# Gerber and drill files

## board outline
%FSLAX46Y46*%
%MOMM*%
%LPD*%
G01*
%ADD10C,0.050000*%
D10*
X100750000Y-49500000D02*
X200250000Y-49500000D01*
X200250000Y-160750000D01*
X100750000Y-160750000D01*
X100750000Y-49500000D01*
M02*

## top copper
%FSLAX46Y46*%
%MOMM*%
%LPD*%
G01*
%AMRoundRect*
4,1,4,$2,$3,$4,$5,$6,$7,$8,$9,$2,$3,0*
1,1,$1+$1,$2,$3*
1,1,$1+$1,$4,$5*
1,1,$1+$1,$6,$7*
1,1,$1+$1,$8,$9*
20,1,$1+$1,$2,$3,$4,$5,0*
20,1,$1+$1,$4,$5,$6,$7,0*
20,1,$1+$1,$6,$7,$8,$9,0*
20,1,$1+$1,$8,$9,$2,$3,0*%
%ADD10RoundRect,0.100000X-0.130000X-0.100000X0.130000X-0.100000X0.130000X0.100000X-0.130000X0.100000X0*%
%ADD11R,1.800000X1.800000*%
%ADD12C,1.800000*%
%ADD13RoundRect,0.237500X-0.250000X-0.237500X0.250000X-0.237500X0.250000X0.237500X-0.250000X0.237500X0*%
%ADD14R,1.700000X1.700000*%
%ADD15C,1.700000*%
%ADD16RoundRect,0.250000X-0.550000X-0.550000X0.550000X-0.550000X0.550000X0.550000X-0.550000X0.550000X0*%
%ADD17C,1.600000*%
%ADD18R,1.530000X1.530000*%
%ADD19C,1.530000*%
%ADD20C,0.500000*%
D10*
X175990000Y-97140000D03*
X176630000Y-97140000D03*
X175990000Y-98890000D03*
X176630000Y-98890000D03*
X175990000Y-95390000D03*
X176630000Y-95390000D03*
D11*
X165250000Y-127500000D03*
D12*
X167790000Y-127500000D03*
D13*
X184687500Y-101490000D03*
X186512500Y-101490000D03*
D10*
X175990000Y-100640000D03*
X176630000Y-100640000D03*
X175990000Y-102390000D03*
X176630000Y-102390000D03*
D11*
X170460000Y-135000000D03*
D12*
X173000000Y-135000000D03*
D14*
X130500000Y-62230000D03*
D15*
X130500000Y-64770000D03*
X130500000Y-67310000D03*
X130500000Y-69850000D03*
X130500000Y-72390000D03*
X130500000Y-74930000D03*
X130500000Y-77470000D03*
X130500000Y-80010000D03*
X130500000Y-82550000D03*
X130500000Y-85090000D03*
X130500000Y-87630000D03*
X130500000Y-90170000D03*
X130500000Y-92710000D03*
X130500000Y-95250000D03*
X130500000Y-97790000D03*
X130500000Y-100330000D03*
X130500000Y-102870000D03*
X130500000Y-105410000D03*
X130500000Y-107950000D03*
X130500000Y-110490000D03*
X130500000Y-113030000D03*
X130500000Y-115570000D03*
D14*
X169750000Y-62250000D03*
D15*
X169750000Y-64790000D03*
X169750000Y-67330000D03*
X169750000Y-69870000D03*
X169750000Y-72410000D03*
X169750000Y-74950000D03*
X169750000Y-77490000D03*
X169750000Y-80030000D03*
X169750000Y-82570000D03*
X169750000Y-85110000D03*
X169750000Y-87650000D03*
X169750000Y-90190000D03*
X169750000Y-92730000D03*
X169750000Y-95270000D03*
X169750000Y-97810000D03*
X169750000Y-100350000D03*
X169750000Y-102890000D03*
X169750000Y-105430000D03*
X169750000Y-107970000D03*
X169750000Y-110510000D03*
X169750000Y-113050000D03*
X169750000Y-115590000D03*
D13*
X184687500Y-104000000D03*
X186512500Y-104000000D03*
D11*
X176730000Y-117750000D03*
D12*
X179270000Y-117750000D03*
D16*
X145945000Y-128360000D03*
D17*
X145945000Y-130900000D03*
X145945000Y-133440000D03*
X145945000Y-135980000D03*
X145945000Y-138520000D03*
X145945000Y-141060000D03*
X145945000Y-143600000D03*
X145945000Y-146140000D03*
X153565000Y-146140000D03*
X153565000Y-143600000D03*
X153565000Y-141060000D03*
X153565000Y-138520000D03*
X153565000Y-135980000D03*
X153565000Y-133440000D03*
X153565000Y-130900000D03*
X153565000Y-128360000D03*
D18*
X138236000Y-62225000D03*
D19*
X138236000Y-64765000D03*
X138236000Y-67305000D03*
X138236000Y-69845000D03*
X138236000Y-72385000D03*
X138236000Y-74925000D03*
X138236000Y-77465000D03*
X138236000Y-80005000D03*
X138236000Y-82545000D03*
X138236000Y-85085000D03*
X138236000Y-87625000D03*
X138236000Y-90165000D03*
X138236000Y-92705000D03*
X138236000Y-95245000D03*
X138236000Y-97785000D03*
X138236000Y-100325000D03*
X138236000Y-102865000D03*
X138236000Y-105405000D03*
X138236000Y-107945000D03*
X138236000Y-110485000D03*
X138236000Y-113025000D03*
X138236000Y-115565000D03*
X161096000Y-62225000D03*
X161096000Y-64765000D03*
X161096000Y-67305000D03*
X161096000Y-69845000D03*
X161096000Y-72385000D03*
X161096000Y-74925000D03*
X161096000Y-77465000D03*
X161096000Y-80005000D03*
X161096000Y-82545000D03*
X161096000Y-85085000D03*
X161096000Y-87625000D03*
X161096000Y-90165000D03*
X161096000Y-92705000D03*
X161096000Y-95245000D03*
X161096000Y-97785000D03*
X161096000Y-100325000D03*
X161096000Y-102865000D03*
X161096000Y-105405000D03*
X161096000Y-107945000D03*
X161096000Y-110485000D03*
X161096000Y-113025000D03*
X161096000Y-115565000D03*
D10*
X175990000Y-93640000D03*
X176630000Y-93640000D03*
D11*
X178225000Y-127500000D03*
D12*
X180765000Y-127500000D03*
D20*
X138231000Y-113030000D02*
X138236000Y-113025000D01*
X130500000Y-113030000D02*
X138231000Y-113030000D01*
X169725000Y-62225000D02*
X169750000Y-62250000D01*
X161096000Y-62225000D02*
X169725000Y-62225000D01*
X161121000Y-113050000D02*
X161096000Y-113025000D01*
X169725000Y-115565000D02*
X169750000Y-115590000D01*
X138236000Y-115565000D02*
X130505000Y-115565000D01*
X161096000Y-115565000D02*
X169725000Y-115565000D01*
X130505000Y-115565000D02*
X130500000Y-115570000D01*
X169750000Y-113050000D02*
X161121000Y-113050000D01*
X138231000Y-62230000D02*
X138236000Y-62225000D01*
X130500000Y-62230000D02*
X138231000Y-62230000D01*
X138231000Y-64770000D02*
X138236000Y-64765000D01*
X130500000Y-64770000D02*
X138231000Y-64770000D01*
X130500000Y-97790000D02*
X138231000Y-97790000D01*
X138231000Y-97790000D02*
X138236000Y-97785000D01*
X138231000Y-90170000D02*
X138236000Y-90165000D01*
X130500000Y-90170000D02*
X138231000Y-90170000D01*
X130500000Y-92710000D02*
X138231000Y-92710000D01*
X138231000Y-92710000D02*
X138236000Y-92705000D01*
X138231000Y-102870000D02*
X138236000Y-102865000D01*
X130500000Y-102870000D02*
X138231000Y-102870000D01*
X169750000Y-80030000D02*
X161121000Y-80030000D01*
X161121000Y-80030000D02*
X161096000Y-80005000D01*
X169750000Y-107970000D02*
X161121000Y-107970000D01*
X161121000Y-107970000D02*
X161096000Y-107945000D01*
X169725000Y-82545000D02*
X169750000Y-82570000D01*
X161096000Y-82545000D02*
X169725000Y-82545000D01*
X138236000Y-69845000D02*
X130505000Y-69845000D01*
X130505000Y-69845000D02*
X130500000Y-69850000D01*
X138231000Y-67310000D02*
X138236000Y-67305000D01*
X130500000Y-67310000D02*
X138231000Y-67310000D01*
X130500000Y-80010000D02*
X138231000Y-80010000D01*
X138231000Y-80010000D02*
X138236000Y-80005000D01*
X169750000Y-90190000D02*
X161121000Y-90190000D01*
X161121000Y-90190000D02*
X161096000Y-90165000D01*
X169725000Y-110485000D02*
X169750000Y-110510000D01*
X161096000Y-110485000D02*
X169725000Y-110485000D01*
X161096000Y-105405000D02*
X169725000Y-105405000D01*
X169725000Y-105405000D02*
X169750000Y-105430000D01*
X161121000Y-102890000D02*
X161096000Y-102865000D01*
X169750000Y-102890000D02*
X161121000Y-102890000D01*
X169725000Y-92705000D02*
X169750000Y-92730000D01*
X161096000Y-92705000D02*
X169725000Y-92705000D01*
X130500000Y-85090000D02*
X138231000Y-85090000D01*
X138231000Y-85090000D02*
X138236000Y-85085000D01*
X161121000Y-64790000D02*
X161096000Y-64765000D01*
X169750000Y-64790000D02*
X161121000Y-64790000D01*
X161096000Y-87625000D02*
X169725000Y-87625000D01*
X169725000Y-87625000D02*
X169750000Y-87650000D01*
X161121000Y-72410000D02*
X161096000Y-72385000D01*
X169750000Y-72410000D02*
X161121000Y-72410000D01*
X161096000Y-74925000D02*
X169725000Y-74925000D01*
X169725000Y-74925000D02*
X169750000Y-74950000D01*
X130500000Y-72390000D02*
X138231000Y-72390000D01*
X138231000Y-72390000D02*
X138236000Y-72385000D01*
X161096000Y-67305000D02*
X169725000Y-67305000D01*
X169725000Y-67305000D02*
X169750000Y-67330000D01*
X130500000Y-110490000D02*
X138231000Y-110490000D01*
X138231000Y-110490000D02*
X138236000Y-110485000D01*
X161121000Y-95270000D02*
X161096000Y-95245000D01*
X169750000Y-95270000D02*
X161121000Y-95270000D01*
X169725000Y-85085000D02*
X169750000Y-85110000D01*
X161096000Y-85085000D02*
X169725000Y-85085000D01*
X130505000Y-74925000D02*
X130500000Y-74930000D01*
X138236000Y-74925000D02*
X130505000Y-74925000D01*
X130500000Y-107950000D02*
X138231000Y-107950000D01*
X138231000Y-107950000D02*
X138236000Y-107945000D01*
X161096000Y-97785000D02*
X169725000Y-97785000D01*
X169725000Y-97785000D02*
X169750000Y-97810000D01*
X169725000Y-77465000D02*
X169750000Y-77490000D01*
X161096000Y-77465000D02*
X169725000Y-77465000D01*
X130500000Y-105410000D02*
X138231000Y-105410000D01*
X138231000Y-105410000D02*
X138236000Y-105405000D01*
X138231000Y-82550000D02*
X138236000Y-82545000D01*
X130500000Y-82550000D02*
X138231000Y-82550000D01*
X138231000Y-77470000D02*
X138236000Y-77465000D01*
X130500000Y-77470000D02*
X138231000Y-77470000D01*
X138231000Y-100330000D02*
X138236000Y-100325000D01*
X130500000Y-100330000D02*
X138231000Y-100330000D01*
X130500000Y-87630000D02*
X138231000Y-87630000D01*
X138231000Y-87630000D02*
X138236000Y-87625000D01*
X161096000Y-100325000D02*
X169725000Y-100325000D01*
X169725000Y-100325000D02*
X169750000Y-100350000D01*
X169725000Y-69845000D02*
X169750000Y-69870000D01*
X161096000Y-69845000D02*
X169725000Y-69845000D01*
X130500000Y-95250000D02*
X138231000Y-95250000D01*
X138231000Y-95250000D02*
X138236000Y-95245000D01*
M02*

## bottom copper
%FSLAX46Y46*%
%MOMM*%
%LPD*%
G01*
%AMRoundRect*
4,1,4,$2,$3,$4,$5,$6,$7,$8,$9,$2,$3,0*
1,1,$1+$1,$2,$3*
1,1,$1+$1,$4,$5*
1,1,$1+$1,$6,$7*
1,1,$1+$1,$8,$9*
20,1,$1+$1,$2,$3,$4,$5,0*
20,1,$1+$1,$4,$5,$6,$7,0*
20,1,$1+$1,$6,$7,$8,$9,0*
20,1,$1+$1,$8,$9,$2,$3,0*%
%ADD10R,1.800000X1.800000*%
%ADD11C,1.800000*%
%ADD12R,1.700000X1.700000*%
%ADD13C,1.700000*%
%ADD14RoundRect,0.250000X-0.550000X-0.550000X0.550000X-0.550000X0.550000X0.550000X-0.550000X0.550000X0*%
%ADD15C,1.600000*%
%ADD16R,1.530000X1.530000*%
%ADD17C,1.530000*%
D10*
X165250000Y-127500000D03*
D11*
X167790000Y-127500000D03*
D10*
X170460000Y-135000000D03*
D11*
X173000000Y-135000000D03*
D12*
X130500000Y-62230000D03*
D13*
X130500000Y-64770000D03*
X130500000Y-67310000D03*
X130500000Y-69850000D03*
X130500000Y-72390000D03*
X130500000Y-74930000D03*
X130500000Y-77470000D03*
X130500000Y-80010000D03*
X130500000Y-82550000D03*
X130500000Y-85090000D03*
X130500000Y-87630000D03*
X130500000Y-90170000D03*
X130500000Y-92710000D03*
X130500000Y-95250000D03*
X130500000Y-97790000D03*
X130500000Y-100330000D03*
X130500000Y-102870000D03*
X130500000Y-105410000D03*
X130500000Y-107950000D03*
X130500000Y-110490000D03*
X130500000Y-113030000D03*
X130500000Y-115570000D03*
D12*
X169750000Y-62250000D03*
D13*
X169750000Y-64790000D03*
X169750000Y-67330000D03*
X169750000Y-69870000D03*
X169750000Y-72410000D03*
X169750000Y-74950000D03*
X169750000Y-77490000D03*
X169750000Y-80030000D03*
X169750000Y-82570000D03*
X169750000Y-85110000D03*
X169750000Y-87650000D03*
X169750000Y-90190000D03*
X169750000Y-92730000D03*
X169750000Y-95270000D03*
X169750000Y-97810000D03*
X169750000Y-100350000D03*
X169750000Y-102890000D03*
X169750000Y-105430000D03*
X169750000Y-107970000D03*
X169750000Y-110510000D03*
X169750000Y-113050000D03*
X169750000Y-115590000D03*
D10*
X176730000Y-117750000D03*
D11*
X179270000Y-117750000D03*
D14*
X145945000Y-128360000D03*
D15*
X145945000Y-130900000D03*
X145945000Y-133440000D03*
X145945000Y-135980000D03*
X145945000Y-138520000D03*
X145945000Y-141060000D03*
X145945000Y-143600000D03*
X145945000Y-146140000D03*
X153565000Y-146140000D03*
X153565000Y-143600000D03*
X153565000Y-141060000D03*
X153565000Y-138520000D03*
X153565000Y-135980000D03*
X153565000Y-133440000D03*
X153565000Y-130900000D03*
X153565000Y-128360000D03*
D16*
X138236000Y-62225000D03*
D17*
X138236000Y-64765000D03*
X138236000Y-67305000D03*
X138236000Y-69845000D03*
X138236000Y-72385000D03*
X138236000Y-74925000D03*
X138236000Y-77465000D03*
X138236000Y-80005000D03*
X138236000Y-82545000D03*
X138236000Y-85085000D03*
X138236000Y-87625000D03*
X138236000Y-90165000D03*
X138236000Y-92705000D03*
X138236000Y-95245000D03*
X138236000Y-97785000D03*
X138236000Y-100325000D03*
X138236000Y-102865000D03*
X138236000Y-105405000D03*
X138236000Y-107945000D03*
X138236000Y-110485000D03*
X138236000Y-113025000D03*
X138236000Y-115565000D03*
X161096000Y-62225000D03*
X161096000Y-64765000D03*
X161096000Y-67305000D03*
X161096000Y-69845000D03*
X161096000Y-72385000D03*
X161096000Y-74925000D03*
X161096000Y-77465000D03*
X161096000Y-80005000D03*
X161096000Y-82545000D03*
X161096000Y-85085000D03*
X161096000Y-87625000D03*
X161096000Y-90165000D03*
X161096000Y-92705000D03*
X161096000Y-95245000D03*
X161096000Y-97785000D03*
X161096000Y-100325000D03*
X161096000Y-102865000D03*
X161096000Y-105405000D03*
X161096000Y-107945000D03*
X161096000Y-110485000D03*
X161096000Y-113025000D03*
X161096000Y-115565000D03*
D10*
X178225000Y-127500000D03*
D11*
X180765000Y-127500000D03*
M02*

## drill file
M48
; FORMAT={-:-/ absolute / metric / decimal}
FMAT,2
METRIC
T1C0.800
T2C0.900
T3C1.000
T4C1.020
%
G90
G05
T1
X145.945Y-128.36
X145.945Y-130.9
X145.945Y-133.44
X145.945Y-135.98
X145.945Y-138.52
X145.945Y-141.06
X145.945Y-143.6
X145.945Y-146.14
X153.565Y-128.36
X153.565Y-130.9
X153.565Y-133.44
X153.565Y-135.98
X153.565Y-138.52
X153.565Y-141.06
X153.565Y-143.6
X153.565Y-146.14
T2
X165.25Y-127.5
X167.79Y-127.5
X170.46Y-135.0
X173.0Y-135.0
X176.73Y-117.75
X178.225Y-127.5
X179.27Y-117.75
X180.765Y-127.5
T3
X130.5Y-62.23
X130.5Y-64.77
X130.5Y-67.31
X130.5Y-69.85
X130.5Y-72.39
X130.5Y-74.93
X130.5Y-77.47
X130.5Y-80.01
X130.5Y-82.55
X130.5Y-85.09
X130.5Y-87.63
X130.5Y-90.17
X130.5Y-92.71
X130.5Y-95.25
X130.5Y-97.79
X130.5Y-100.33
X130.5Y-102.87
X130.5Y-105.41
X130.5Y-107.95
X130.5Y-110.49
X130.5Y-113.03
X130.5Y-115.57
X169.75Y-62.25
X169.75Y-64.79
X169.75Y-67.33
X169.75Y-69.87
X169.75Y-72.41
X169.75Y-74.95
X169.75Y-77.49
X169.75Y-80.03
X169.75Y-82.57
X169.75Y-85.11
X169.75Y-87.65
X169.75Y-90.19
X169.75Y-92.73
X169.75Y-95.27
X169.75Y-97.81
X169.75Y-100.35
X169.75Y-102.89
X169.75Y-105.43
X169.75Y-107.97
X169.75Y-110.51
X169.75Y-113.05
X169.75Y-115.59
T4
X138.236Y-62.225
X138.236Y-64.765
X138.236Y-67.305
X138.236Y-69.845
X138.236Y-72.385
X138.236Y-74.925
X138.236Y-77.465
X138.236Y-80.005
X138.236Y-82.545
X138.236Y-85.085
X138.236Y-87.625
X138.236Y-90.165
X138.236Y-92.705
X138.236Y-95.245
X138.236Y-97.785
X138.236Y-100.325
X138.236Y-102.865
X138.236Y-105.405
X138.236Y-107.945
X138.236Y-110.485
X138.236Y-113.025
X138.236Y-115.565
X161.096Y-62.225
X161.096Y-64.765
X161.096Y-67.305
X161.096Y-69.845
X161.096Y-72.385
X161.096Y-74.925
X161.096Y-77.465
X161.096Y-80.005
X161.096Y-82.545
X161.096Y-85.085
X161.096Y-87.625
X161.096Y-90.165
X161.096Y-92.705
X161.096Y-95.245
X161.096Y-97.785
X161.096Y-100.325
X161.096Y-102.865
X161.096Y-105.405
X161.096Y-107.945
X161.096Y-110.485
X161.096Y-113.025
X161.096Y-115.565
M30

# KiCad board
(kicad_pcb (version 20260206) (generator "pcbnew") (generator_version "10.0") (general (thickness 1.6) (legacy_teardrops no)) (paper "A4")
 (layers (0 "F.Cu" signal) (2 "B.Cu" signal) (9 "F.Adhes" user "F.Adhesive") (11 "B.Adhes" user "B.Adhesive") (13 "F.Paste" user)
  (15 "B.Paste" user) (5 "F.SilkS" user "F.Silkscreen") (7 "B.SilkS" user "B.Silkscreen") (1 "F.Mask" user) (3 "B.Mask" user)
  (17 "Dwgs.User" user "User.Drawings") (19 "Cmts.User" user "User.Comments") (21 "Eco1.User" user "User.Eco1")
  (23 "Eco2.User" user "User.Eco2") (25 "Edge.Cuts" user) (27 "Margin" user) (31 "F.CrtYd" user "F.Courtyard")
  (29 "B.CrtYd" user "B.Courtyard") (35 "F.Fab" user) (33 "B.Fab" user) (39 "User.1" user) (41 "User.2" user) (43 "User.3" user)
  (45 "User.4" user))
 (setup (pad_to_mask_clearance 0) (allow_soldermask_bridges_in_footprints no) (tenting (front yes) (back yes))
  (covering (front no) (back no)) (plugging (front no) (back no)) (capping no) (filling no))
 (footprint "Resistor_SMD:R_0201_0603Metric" (layer "F.Cu") (at 176.31 97.14)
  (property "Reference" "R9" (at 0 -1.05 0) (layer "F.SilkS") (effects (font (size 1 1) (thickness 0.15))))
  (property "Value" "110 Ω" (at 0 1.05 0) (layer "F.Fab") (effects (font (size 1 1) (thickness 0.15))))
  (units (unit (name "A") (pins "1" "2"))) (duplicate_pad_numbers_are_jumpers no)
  (pad "" smd roundrect (at -0.345 0) (size 0.318 0.36) (layers "F.Paste") (roundrect_rratio 0.25))
  (pad "" smd roundrect (at 0.345 0) (size 0.318 0.36) (layers "F.Paste") (roundrect_rratio 0.25))
  (pad "1" smd roundrect (at -0.32 0) (size 0.46 0.4) (layers "F.Cu" "F.Mask") (roundrect_rratio 0.25) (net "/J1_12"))
  (pad "2" smd roundrect (at 0.32 0) (size 0.46 0.4) (layers "F.Cu" "F.Mask") (roundrect_rratio 0.25) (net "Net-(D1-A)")))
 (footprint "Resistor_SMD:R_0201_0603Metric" (layer "F.Cu") (at 176.31 98.89)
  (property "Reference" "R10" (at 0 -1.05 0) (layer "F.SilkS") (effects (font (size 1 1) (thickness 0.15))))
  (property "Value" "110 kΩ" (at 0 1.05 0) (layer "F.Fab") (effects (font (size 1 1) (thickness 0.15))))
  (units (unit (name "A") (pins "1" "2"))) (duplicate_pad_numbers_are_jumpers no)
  (pad "" smd roundrect (at -0.345 0) (size 0.318 0.36) (layers "F.Paste") (roundrect_rratio 0.25))
  (pad "" smd roundrect (at 0.345 0) (size 0.318 0.36) (layers "F.Paste") (roundrect_rratio 0.25))
  (pad "1" smd roundrect (at -0.32 0) (size 0.46 0.4) (layers "F.Cu" "F.Mask") (roundrect_rratio 0.25) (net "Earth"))
  (pad "2" smd roundrect (at 0.32 0) (size 0.46 0.4) (layers "F.Cu" "F.Mask") (roundrect_rratio 0.25) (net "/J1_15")))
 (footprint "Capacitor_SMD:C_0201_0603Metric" (layer "F.Cu") (at 176.31 95.39)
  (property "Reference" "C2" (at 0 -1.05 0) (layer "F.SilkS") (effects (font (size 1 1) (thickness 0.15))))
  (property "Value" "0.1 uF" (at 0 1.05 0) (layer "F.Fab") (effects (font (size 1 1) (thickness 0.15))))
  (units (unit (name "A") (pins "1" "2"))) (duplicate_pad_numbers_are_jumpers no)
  (pad "" smd roundrect (at -0.345 0) (size 0.318 0.36) (layers "F.Paste") (roundrect_rratio 0.25))
  (pad "" smd roundrect (at 0.345 0) (size 0.318 0.36) (layers "F.Paste") (roundrect_rratio 0.25))
  (pad "1" smd roundrect (at -0.32 0) (size 0.46 0.4) (layers "F.Cu" "F.Mask") (roundrect_rratio 0.25) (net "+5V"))
  (pad "2" smd roundrect (at 0.32 0) (size 0.46 0.4) (layers "F.Cu" "F.Mask") (roundrect_rratio 0.25) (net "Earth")))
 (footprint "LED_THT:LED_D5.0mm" (layer "F.Cu") (at 165.25 127.5)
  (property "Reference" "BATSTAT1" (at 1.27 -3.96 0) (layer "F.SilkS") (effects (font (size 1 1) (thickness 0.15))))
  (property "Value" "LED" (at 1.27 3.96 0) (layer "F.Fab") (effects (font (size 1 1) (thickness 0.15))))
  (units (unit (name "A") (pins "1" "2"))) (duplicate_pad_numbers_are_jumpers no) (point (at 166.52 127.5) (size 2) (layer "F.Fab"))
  (pad "1" thru_hole rect (at 0 0) (size 1.8 1.8) (drill 0.9) (layers "*.Cu" "*.Mask") (remove_unused_layers no) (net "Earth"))
  (pad "2" thru_hole circle (at 2.54 0) (size 1.8 1.8) (drill 0.9) (layers "*.Cu" "*.Mask") (remove_unused_layers no)
   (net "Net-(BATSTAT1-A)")))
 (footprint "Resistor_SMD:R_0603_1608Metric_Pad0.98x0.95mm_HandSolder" (layer "F.Cu") (at 185.6 101.49)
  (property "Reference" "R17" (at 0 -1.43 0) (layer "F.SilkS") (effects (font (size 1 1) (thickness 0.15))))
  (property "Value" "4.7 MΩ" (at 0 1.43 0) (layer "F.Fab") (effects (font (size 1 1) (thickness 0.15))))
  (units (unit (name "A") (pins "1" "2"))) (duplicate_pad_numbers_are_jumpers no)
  (pad "1" smd roundrect (at -0.9125 0) (size 0.975 0.95) (layers "F.Cu" "F.Mask" "F.Paste") (roundrect_rratio 0.25) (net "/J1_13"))
  (pad "2" smd roundrect (at 0.9125 0) (size 0.975 0.95) (layers "F.Cu" "F.Mask" "F.Paste") (roundrect_rratio 0.25) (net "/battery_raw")))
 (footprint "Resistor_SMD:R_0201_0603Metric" (layer "F.Cu") (at 176.31 100.64)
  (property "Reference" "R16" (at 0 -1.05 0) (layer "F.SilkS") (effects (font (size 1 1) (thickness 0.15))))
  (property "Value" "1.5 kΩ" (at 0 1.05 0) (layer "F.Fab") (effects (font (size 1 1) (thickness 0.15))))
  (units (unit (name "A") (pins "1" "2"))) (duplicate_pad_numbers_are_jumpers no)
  (pad "" smd roundrect (at -0.345 0) (size 0.318 0.36) (layers "F.Paste") (roundrect_rratio 0.25))
  (pad "" smd roundrect (at 0.345 0) (size 0.318 0.36) (layers "F.Paste") (roundrect_rratio 0.25))
  (pad "1" smd roundrect (at -0.32 0) (size 0.46 0.4) (layers "F.Cu" "F.Mask") (roundrect_rratio 0.25) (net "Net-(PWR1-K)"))
  (pad "2" smd roundrect (at 0.32 0) (size 0.46 0.4) (layers "F.Cu" "F.Mask") (roundrect_rratio 0.25) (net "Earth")))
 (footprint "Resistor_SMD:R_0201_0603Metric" (layer "F.Cu") (at 176.31 102.39)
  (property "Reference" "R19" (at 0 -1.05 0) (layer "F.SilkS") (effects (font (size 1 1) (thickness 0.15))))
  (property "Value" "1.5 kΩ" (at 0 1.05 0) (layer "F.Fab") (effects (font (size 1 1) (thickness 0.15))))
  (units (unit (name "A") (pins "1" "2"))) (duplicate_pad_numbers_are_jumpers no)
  (pad "" smd roundrect (at -0.345 0) (size 0.318 0.36) (layers "F.Paste") (roundrect_rratio 0.25))
  (pad "" smd roundrect (at 0.345 0) (size 0.318 0.36) (layers "F.Paste") (roundrect_rratio 0.25))
  (pad "1" smd roundrect (at -0.32 0) (size 0.46 0.4) (layers "F.Cu" "F.Mask") (roundrect_rratio 0.25) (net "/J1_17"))
  (pad "2" smd roundrect (at 0.32 0) (size 0.46 0.4) (layers "F.Cu" "F.Mask") (roundrect_rratio 0.25) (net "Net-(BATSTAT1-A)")))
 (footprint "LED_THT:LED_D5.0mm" (layer "F.Cu") (at 170.46 135)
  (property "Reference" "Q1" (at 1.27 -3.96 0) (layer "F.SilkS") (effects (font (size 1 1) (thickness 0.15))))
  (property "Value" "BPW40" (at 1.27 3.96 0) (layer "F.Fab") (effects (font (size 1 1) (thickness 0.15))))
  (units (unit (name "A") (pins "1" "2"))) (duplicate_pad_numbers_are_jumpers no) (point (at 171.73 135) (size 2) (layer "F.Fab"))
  (pad "1" thru_hole rect (at 0 0) (size 1.8 1.8) (drill 0.9) (layers "*.Cu" "*.Mask") (remove_unused_layers no) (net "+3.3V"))
  (pad "2" thru_hole circle (at 2.54 0) (size 1.8 1.8) (drill 0.9) (layers "*.Cu" "*.Mask") (remove_unused_layers no) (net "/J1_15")))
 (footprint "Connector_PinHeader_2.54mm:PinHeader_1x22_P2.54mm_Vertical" (layer "F.Cu") (at 130.5 62.23)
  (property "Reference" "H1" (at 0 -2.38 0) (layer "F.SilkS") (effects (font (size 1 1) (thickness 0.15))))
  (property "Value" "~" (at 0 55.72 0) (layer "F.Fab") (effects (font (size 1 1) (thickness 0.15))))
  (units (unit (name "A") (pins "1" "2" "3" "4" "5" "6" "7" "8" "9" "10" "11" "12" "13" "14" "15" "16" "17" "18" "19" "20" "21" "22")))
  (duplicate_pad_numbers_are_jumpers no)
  (pad "1" thru_hole rect (at 0 0) (size 1.7 1.7) (drill 1) (layers "*.Cu" "*.Mask") (remove_unused_layers no) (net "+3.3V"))
  (pad "2" thru_hole circle (at 0 2.54) (size 1.7 1.7) (drill 1) (layers "*.Cu" "*.Mask") (remove_unused_layers no) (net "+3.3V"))
  (pad "3" thru_hole circle (at 0 5.08) (size 1.7 1.7) (drill 1) (layers "*.Cu" "*.Mask") (remove_unused_layers no) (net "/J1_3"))
  (pad "4" thru_hole circle (at 0 7.62) (size 1.7 1.7) (drill 1) (layers "*.Cu" "*.Mask") (remove_unused_layers no) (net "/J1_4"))
  (pad "5" thru_hole circle (at 0 10.16) (size 1.7 1.7) (drill 1) (layers "*.Cu" "*.Mask") (remove_unused_layers no) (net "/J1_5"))
  (pad "6" thru_hole circle (at 0 12.7) (size 1.7 1.7) (drill 1) (layers "*.Cu" "*.Mask") (remove_unused_layers no) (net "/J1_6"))
  (pad "7" thru_hole circle (at 0 15.24) (size 1.7 1.7) (drill 1) (layers "*.Cu" "*.Mask") (remove_unused_layers no) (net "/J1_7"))
  (pad "8" thru_hole circle (at 0 17.78) (size 1.7 1.7) (drill 1) (layers "*.Cu" "*.Mask") (remove_unused_layers no) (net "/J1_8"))
  (pad "9" thru_hole circle (at 0 20.32) (size 1.7 1.7) (drill 1) (layers "*.Cu" "*.Mask") (remove_unused_layers no) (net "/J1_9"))
  (pad "10" thru_hole circle (at 0 22.86) (size 1.7 1.7) (drill 1) (layers "*.Cu" "*.Mask") (remove_unused_layers no) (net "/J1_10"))
  (pad "11" thru_hole circle (at 0 25.4) (size 1.7 1.7) (drill 1) (layers "*.Cu" "*.Mask") (remove_unused_layers no) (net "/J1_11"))
  (pad "12" thru_hole circle (at 0 27.94) (size 1.7 1.7) (drill 1) (layers "*.Cu" "*.Mask") (remove_unused_layers no) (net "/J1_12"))
  (pad "13" thru_hole circle (at 0 30.48) (size 1.7 1.7) (drill 1) (layers "*.Cu" "*.Mask") (remove_unused_layers no) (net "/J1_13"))
  (pad "14" thru_hole circle (at 0 33.02) (size 1.7 1.7) (drill 1) (layers "*.Cu" "*.Mask") (remove_unused_layers no) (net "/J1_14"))
  (pad "15" thru_hole circle (at 0 35.56) (size 1.7 1.7) (drill 1) (layers "*.Cu" "*.Mask") (remove_unused_layers no) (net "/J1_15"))
  (pad "16" thru_hole circle (at 0 38.1) (size 1.7 1.7) (drill 1) (layers "*.Cu" "*.Mask") (remove_unused_layers no) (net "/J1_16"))
  (pad "17" thru_hole circle (at 0 40.64) (size 1.7 1.7) (drill 1) (layers "*.Cu" "*.Mask") (remove_unused_layers no) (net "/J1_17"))
  (pad "18" thru_hole circle (at 0 43.18) (size 1.7 1.7) (drill 1) (layers "*.Cu" "*.Mask") (remove_unused_layers no) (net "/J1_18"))
  (pad "19" thru_hole circle (at 0 45.72) (size 1.7 1.7) (drill 1) (layers "*.Cu" "*.Mask") (remove_unused_layers no) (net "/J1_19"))
  (pad "20" thru_hole circle (at 0 48.26) (size 1.7 1.7) (drill 1) (layers "*.Cu" "*.Mask") (remove_unused_layers no) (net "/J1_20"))
  (pad "21" thru_hole circle (at 0 50.8) (size 1.7 1.7) (drill 1) (layers "*.Cu" "*.Mask") (remove_unused_layers no) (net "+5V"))
  (pad "22" thru_hole circle (at 0 53.34) (size 1.7 1.7) (drill 1) (layers "*.Cu" "*.Mask") (remove_unused_layers no) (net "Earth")))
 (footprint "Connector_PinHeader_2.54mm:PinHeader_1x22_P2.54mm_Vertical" (layer "F.Cu") (at 169.75 62.25)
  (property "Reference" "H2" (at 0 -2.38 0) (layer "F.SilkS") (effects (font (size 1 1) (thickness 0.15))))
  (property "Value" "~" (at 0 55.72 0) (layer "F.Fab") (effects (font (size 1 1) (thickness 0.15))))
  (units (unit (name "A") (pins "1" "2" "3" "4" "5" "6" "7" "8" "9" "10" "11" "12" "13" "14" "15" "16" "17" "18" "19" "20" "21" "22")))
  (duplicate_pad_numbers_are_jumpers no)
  (pad "1" thru_hole rect (at 0 0) (size 1.7 1.7) (drill 1) (layers "*.Cu" "*.Mask") (remove_unused_layers no) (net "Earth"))
  (pad "2" thru_hole circle (at 0 2.54) (size 1.7 1.7) (drill 1) (layers "*.Cu" "*.Mask") (remove_unused_layers no) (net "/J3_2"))
  (pad "3" thru_hole circle (at 0 5.08) (size 1.7 1.7) (drill 1) (layers "*.Cu" "*.Mask") (remove_unused_layers no) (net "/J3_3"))
  (pad "4" thru_hole circle (at 0 7.62) (size 1.7 1.7) (drill 1) (layers "*.Cu" "*.Mask") (remove_unused_layers no) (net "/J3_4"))
  (pad "5" thru_hole circle (at 0 10.16) (size 1.7 1.7) (drill 1) (layers "*.Cu" "*.Mask") (remove_unused_layers no) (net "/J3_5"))
  (pad "6" thru_hole circle (at 0 12.7) (size 1.7 1.7) (drill 1) (layers "*.Cu" "*.Mask") (remove_unused_layers no) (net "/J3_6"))
  (pad "7" thru_hole circle (at 0 15.24) (size 1.7 1.7) (drill 1) (layers "*.Cu" "*.Mask") (remove_unused_layers no) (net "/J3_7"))
  (pad "8" thru_hole circle (at 0 17.78) (size 1.7 1.7) (drill 1) (layers "*.Cu" "*.Mask") (remove_unused_layers no) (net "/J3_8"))
  (pad "9" thru_hole circle (at 0 20.32) (size 1.7 1.7) (drill 1) (layers "*.Cu" "*.Mask") (remove_unused_layers no) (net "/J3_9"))
  (pad "10" thru_hole circle (at 0 22.86) (size 1.7 1.7) (drill 1) (layers "*.Cu" "*.Mask") (remove_unused_layers no) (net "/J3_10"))
  (pad "11" thru_hole circle (at 0 25.4) (size 1.7 1.7) (drill 1) (layers "*.Cu" "*.Mask") (remove_unused_layers no) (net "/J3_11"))
  (pad "12" thru_hole circle (at 0 27.94) (size 1.7 1.7) (drill 1) (layers "*.Cu" "*.Mask") (remove_unused_layers no) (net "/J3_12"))
  (pad "13" thru_hole circle (at 0 30.48) (size 1.7 1.7) (drill 1) (layers "*.Cu" "*.Mask") (remove_unused_layers no) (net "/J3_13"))
  (pad "14" thru_hole circle (at 0 33.02) (size 1.7 1.7) (drill 1) (layers "*.Cu" "*.Mask") (remove_unused_layers no) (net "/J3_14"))
  (pad "15" thru_hole circle (at 0 35.56) (size 1.7 1.7) (drill 1) (layers "*.Cu" "*.Mask") (remove_unused_layers no) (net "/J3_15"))
  (pad "16" thru_hole circle (at 0 38.1) (size 1.7 1.7) (drill 1) (layers "*.Cu" "*.Mask") (remove_unused_layers no) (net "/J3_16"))
  (pad "17" thru_hole circle (at 0 40.64) (size 1.7 1.7) (drill 1) (layers "*.Cu" "*.Mask") (remove_unused_layers no) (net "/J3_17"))
  (pad "18" thru_hole circle (at 0 43.18) (size 1.7 1.7) (drill 1) (layers "*.Cu" "*.Mask") (remove_unused_layers no) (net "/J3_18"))
  (pad "19" thru_hole circle (at 0 45.72) (size 1.7 1.7) (drill 1) (layers "*.Cu" "*.Mask") (remove_unused_layers no) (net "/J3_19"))
  (pad "20" thru_hole circle (at 0 48.26) (size 1.7 1.7) (drill 1) (layers "*.Cu" "*.Mask") (remove_unused_layers no) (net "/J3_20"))
  (pad "21" thru_hole circle (at 0 50.8) (size 1.7 1.7) (drill 1) (layers "*.Cu" "*.Mask") (remove_unused_layers no) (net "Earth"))
  (pad "22" thru_hole circle (at 0 53.34) (size 1.7 1.7) (drill 1) (layers "*.Cu" "*.Mask") (remove_unused_layers no) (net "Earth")))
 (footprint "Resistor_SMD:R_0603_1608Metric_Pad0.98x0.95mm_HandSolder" (layer "F.Cu") (at 185.6 104)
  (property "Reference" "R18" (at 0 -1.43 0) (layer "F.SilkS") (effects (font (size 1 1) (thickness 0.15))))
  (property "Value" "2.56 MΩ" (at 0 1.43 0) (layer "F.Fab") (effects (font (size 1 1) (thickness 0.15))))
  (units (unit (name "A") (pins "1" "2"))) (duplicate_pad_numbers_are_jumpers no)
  (pad "1" smd roundrect (at -0.9125 0) (size 0.975 0.95) (layers "F.Cu" "F.Mask" "F.Paste") (roundrect_rratio 0.25) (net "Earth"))
  (pad "2" smd roundrect (at 0.9125 0) (size 0.975 0.95) (layers "F.Cu" "F.Mask" "F.Paste") (roundrect_rratio 0.25) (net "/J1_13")))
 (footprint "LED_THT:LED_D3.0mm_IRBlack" (layer "F.Cu") (at 176.73 117.75)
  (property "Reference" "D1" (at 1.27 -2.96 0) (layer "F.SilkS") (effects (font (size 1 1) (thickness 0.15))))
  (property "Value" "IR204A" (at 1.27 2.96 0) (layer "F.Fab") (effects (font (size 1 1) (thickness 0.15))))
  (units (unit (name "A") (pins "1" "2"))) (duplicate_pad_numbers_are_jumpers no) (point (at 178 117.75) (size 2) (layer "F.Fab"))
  (pad "1" thru_hole rect (at 0 0) (size 1.8 1.8) (drill 0.9) (layers "*.Cu" "*.Mask") (remove_unused_layers no) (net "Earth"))
  (pad "2" thru_hole circle (at 2.54 0) (size 1.8 1.8) (drill 0.9) (layers "*.Cu" "*.Mask") (remove_unused_layers no) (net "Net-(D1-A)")))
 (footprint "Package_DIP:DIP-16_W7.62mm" (layer "F.Cu") (at 145.945 128.36)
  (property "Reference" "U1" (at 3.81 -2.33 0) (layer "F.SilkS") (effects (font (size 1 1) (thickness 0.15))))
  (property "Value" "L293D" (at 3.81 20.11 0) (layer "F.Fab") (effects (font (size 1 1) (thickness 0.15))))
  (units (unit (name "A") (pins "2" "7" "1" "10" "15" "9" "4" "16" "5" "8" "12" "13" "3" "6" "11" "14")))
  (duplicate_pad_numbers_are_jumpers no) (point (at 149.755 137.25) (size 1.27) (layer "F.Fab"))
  (pad "1" thru_hole roundrect (at 0 0) (size 1.6 1.6) (drill 0.8) (layers "*.Cu" "*.Mask") (remove_unused_layers no)
   (roundrect_rratio 0.15625) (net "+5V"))
  (pad "2" thru_hole circle (at 0 2.54) (size 1.6 1.6) (drill 0.8) (layers "*.Cu" "*.Mask") (remove_unused_layers no) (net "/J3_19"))
  (pad "3" thru_hole circle (at 0 5.08) (size 1.6 1.6) (drill 0.8) (layers "*.Cu" "*.Mask") (remove_unused_layers no)
   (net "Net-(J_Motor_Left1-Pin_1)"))
  (pad "4" thru_hole circle (at 0 7.62) (size 1.6 1.6) (drill 0.8) (layers "*.Cu" "*.Mask") (remove_unused_layers no) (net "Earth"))
  (pad "5" thru_hole circle (at 0 10.16) (size 1.6 1.6) (drill 0.8) (layers "*.Cu" "*.Mask") (remove_unused_layers no) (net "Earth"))
  (pad "6" thru_hole circle (at 0 12.7) (size 1.6 1.6) (drill 0.8) (layers "*.Cu" "*.Mask") (remove_unused_layers no)
   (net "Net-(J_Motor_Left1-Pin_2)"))
  (pad "7" thru_hole circle (at 0 15.24) (size 1.6 1.6) (drill 0.8) (layers "*.Cu" "*.Mask") (remove_unused_layers no) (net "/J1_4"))
  (pad "8" thru_hole circle (at 0 17.78) (size 1.6 1.6) (drill 0.8) (layers "*.Cu" "*.Mask") (remove_unused_layers no) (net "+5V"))
  (pad "9" thru_hole circle (at 7.62 17.78) (size 1.6 1.6) (drill 0.8) (layers "*.Cu" "*.Mask") (remove_unused_layers no) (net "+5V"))
  (pad "10" thru_hole circle (at 7.62 15.24) (size 1.6 1.6) (drill 0.8) (layers "*.Cu" "*.Mask") (remove_unused_layers no) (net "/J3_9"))
  (pad "11" thru_hole circle (at 7.62 12.7) (size 1.6 1.6) (drill 0.8) (layers "*.Cu" "*.Mask") (remove_unused_layers no)
   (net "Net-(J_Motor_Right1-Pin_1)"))
  (pad "12" thru_hole circle (at 7.62 10.16) (size 1.6 1.6) (drill 0.8) (layers "*.Cu" "*.Mask") (remove_unused_layers no) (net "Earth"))
  (pad "13" thru_hole circle (at 7.62 7.62) (size 1.6 1.6) (drill 0.8) (layers "*.Cu" "*.Mask") (remove_unused_layers no) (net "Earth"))
  (pad "14" thru_hole circle (at 7.62 5.08) (size 1.6 1.6) (drill 0.8) (layers "*.Cu" "*.Mask") (remove_unused_layers no)
   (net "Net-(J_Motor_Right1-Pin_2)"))
  (pad "15" thru_hole circle (at 7.62 2.54) (size 1.6 1.6) (drill 0.8) (layers "*.Cu" "*.Mask") (remove_unused_layers no) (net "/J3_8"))
  (pad "16" thru_hole circle (at 7.62 0) (size 1.6 1.6) (drill 0.8) (layers "*.Cu" "*.Mask") (remove_unused_layers no) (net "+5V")))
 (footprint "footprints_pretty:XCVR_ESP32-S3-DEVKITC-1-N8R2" (layer "F.Cu") (at 149.666 92.195)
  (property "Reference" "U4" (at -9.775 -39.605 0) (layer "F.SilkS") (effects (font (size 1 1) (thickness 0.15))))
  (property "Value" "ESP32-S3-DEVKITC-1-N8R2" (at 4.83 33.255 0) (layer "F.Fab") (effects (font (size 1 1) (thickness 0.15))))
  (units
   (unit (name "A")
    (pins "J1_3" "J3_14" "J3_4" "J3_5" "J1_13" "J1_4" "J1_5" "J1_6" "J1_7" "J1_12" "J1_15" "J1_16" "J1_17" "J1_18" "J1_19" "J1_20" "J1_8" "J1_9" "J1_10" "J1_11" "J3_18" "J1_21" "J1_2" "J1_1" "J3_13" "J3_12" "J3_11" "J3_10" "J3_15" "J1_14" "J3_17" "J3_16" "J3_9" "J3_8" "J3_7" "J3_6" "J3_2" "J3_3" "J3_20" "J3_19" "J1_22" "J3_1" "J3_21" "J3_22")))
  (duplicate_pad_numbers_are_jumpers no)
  (pad "J1_1" thru_hole rect (at -11.43 -29.97) (size 1.53 1.53) (drill 1.02) (layers "*.Cu" "*.Mask") (remove_unused_layers no)
   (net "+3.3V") (solder_mask_margin 0.102))
  (pad "J1_2" thru_hole circle (at -11.43 -27.43) (size 1.53 1.53) (drill 1.02) (layers "*.Cu" "*.Mask") (remove_unused_layers no)
   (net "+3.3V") (solder_mask_margin 0.102))
  (pad "J1_3" thru_hole circle (at -11.43 -24.89) (size 1.53 1.53) (drill 1.02) (layers "*.Cu" "*.Mask") (remove_unused_layers no)
   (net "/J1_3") (solder_mask_margin 0.102))
  (pad "J1_4" thru_hole circle (at -11.43 -22.35) (size 1.53 1.53) (drill 1.02) (layers "*.Cu" "*.Mask") (remove_unused_layers no)
   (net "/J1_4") (solder_mask_margin 0.102))
  (pad "J1_5" thru_hole circle (at -11.43 -19.81) (size 1.53 1.53) (drill 1.02) (layers "*.Cu" "*.Mask") (remove_unused_layers no)
   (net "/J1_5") (solder_mask_margin 0.102))
  (pad "J1_6" thru_hole circle (at -11.43 -17.27) (size 1.53 1.53) (drill 1.02) (layers "*.Cu" "*.Mask") (remove_unused_layers no)
   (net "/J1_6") (solder_mask_margin 0.102))
  (pad "J1_7" thru_hole circle (at -11.43 -14.73) (size 1.53 1.53) (drill 1.02) (layers "*.Cu" "*.Mask") (remove_unused_layers no)
   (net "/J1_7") (solder_mask_margin 0.102))
  (pad "J1_8" thru_hole circle (at -11.43 -12.19) (size 1.53 1.53) (drill 1.02) (layers "*.Cu" "*.Mask") (remove_unused_layers no)
   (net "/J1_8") (solder_mask_margin 0.102))
  (pad "J1_9" thru_hole circle (at -11.43 -9.65) (size 1.53 1.53) (drill 1.02) (layers "*.Cu" "*.Mask") (remove_unused_layers no)
   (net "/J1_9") (solder_mask_margin 0.102))
  (pad "J1_10" thru_hole circle (at -11.43 -7.11) (size 1.53 1.53) (drill 1.02) (layers "*.Cu" "*.Mask") (remove_unused_layers no)
   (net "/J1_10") (solder_mask_margin 0.102))
  (pad "J1_11" thru_hole circle (at -11.43 -4.57) (size 1.53 1.53) (drill 1.02) (layers "*.Cu" "*.Mask") (remove_unused_layers no)
   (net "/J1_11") (solder_mask_margin 0.102))
  (pad "J1_12" thru_hole circle (at -11.43 -2.03) (size 1.53 1.53) (drill 1.02) (layers "*.Cu" "*.Mask") (remove_unused_layers no)
   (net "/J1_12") (solder_mask_margin 0.102))
  (pad "J1_13" thru_hole circle (at -11.43 0.51) (size 1.53 1.53) (drill 1.02) (layers "*.Cu" "*.Mask") (remove_unused_layers no)
   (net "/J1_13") (solder_mask_margin 0.102))
  (pad "J1_14" thru_hole circle (at -11.43 3.05) (size 1.53 1.53) (drill 1.02) (layers "*.Cu" "*.Mask") (remove_unused_layers no)
   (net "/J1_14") (solder_mask_margin 0.102))
  (pad "J1_15" thru_hole circle (at -11.43 5.59) (size 1.53 1.53) (drill 1.02) (layers "*.Cu" "*.Mask") (remove_unused_layers no)
   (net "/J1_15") (solder_mask_margin 0.102))
  (pad "J1_16" thru_hole circle (at -11.43 8.13) (size 1.53 1.53) (drill 1.02) (layers "*.Cu" "*.Mask") (remove_unused_layers no)
   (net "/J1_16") (solder_mask_margin 0.102))
  (pad "J1_17" thru_hole circle (at -11.43 10.67) (size 1.53 1.53) (drill 1.02) (layers "*.Cu" "*.Mask") (remove_unused_layers no)
   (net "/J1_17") (solder_mask_margin 0.102))
  (pad "J1_18" thru_hole circle (at -11.43 13.21) (size 1.53 1.53) (drill 1.02) (layers "*.Cu" "*.Mask") (remove_unused_layers no)
   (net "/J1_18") (solder_mask_margin 0.102))
  (pad "J1_19" thru_hole circle (at -11.43 15.75) (size 1.53 1.53) (drill 1.02) (layers "*.Cu" "*.Mask") (remove_unused_layers no)
   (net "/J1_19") (solder_mask_margin 0.102))
  (pad "J1_20" thru_hole circle (at -11.43 18.29) (size 1.53 1.53) (drill 1.02) (layers "*.Cu" "*.Mask") (remove_unused_layers no)
   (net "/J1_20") (solder_mask_margin 0.102))
  (pad "J1_21" thru_hole circle (at -11.43 20.83) (size 1.53 1.53) (drill 1.02) (layers "*.Cu" "*.Mask") (remove_unused_layers no)
   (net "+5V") (solder_mask_margin 0.102))
  (pad "J1_22" thru_hole circle (at -11.43 23.37) (size 1.53 1.53) (drill 1.02) (layers "*.Cu" "*.Mask") (remove_unused_layers no)
   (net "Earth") (solder_mask_margin 0.102))
  (pad "J3_1" thru_hole circle (at 11.43 -29.97) (size 1.53 1.53) (drill 1.02) (layers "*.Cu" "*.Mask") (remove_unused_layers no)
   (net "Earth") (solder_mask_margin 0.102))
  (pad "J3_2" thru_hole circle (at 11.43 -27.43) (size 1.53 1.53) (drill 1.02) (layers "*.Cu" "*.Mask") (remove_unused_layers no)
   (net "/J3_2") (solder_mask_margin 0.102))
  (pad "J3_3" thru_hole circle (at 11.43 -24.89) (size 1.53 1.53) (drill 1.02) (layers "*.Cu" "*.Mask") (remove_unused_layers no)
   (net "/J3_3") (solder_mask_margin 0.102))
  (pad "J3_4" thru_hole circle (at 11.43 -22.35) (size 1.53 1.53) (drill 1.02) (layers "*.Cu" "*.Mask") (remove_unused_layers no)
   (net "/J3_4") (solder_mask_margin 0.102))
  (pad "J3_5" thru_hole circle (at 11.43 -19.81) (size 1.53 1.53) (drill 1.02) (layers "*.Cu" "*.Mask") (remove_unused_layers no)
   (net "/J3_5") (solder_mask_margin 0.102))
  (pad "J3_6" thru_hole circle (at 11.43 -17.27) (size 1.53 1.53) (drill 1.02) (layers "*.Cu" "*.Mask") (remove_unused_layers no)
   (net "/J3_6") (solder_mask_margin 0.102))
  (pad "J3_7" thru_hole circle (at 11.43 -14.73) (size 1.53 1.53) (drill 1.02) (layers "*.Cu" "*.Mask") (remove_unused_layers no)
   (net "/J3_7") (solder_mask_margin 0.102))
  (pad "J3_8" thru_hole circle (at 11.43 -12.19) (size 1.53 1.53) (drill 1.02) (layers "*.Cu" "*.Mask") (remove_unused_layers no)
   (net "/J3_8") (solder_mask_margin 0.102))
  (pad "J3_9" thru_hole circle (at 11.43 -9.65) (size 1.53 1.53) (drill 1.02) (layers "*.Cu" "*.Mask") (remove_unused_layers no)
   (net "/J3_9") (solder_mask_margin 0.102))
  (pad "J3_10" thru_hole circle (at 11.43 -7.11) (size 1.53 1.53) (drill 1.02) (layers "*.Cu" "*.Mask") (remove_unused_layers no)
   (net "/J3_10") (solder_mask_margin 0.102))
  (pad "J3_11" thru_hole circle (at 11.43 -4.57) (size 1.53 1.53) (drill 1.02) (layers "*.Cu" "*.Mask") (remove_unused_layers no)
   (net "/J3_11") (solder_mask_margin 0.102))
  (pad "J3_12" thru_hole circle (at 11.43 -2.03) (size 1.53 1.53) (drill 1.02) (layers "*.Cu" "*.Mask") (remove_unused_layers no)
   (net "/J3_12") (solder_mask_margin 0.102))
  (pad "J3_13" thru_hole circle (at 11.43 0.51) (size 1.53 1.53) (drill 1.02) (layers "*.Cu" "*.Mask") (remove_unused_layers no)
   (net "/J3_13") (solder_mask_margin 0.102))
  (pad "J3_14" thru_hole circle (at 11.43 3.05) (size 1.53 1.53) (drill 1.02) (layers "*.Cu" "*.Mask") (remove_unused_layers no)
   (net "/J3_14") (solder_mask_margin 0.102))
  (pad "J3_15" thru_hole circle (at 11.43 5.59) (size 1.53 1.53) (drill 1.02) (layers "*.Cu" "*.Mask") (remove_unused_layers no)
   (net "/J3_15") (solder_mask_margin 0.102))
  (pad "J3_16" thru_hole circle (at 11.43 8.13) (size 1.53 1.53) (drill 1.02) (layers "*.Cu" "*.Mask") (remove_unused_layers no)
   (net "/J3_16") (solder_mask_margin 0.102))
  (pad "J3_17" thru_hole circle (at 11.43 10.67) (size 1.53 1.53) (drill 1.02) (layers "*.Cu" "*.Mask") (remove_unused_layers no)
   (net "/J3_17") (solder_mask_margin 0.102))
  (pad "J3_18" thru_hole circle (at 11.43 13.21) (size 1.53 1.53) (drill 1.02) (layers "*.Cu" "*.Mask") (remove_unused_layers no)
   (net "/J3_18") (solder_mask_margin 0.102))
  (pad "J3_19" thru_hole circle (at 11.43 15.75) (size 1.53 1.53) (drill 1.02) (layers "*.Cu" "*.Mask") (remove_unused_layers no)
   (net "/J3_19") (solder_mask_margin 0.102))
  (pad "J3_20" thru_hole circle (at 11.43 18.29) (size 1.53 1.53) (drill 1.02) (layers "*.Cu" "*.Mask") (remove_unused_layers no)
   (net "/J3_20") (solder_mask_margin 0.102))
  (pad "J3_21" thru_hole circle (at 11.43 20.83) (size 1.53 1.53) (drill 1.02) (layers "*.Cu" "*.Mask") (remove_unused_layers no)
   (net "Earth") (solder_mask_margin 0.102))
  (pad "J3_22" thru_hole circle (at 11.43 23.37) (size 1.53 1.53) (drill 1.02) (layers "*.Cu" "*.Mask") (remove_unused_layers no)
   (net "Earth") (solder_mask_margin 0.102)))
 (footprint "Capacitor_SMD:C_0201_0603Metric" (layer "F.Cu") (at 176.31 93.64)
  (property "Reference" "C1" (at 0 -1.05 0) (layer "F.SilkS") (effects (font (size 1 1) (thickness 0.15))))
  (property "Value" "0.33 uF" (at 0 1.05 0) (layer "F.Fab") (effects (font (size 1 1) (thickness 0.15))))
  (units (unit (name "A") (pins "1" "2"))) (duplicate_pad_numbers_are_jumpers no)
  (pad "" smd roundrect (at -0.345 0) (size 0.318 0.36) (layers "F.Paste") (roundrect_rratio 0.25))
  (pad "" smd roundrect (at 0.345 0) (size 0.318 0.36) (layers "F.Paste") (roundrect_rratio 0.25))
  (pad "1" smd roundrect (at -0.32 0) (size 0.46 0.4) (layers "F.Cu" "F.Mask") (roundrect_rratio 0.25) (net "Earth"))
  (pad "2" smd roundrect (at 0.32 0) (size 0.46 0.4) (layers "F.Cu" "F.Mask") (roundrect_rratio 0.25) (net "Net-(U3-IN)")))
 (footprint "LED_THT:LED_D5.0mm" (layer "F.Cu") (at 178.225 127.5)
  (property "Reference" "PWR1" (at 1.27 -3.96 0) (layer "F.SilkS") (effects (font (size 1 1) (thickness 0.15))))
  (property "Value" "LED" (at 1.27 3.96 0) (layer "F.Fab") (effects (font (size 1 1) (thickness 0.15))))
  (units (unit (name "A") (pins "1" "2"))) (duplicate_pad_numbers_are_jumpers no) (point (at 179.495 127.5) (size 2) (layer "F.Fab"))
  (pad "1" thru_hole rect (at 0 0) (size 1.8 1.8) (drill 0.9) (layers "*.Cu" "*.Mask") (remove_unused_layers no) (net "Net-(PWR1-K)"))
  (pad "2" thru_hole circle (at 2.54 0) (size 1.8 1.8) (drill 0.9) (layers "*.Cu" "*.Mask") (remove_unused_layers no) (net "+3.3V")))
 (gr_rect (start 100.75 49.5) (end 200.25 160.75) (stroke (width 0.05) (type default)) (fill no) (layer "Edge.Cuts"))
 (segment (start 138.231 113.03) (end 138.236 113.025) (width 0.5) (layer "F.Cu") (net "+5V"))
 (segment (start 130.5 113.03) (end 138.231 113.03) (width 0.5) (layer "F.Cu") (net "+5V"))
 (segment (start 169.725 62.225) (end 169.75 62.25) (width 0.5) (layer "F.Cu") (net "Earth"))
 (segment (start 161.096 62.225) (end 169.725 62.225) (width 0.5) (layer "F.Cu") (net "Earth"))
 (segment (start 161.121 113.05) (end 161.096 113.025) (width 0.5) (layer "F.Cu") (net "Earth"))
 (segment (start 169.725 115.565) (end 169.75 115.59) (width 0.5) (layer "F.Cu") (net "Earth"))
 (segment (start 138.236 115.565) (end 130.505 115.565) (width 0.5) (layer "F.Cu") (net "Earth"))
 (segment (start 161.096 115.565) (end 169.725 115.565) (width 0.5) (layer "F.Cu") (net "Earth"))
 (segment (start 130.505 115.565) (end 130.5 115.57) (width 0.5) (layer "F.Cu") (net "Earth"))
 (segment (start 169.75 113.05) (end 161.121 113.05) (width 0.5) (layer "F.Cu") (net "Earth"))
 (segment (start 138.231 62.23) (end 138.236 62.225) (width 0.5) (layer "F.Cu") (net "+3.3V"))
 (segment (start 130.5 62.23) (end 138.231 62.23) (width 0.5) (layer "F.Cu") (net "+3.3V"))
 (segment (start 138.231 64.77) (end 138.236 64.765) (width 0.5) (layer "F.Cu") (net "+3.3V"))
 (segment (start 130.5 64.77) (end 138.231 64.77) (width 0.5) (layer "F.Cu") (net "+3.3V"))
 (segment (start 130.5 97.79) (end 138.231 97.79) (width 0.5) (layer "F.Cu") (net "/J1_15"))
 (segment (start 138.231 97.79) (end 138.236 97.785) (width 0.5) (layer "F.Cu") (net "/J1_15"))
 (segment (start 138.231 90.17) (end 138.236 90.165) (width 0.5) (layer "F.Cu") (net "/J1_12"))
 (segment (start 130.5 90.17) (end 138.231 90.17) (width 0.5) (layer "F.Cu") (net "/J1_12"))
 (segment (start 130.5 92.71) (end 138.231 92.71) (width 0.5) (layer "F.Cu") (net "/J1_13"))
 (segment (start 138.231 92.71) (end 138.236 92.705) (width 0.5) (layer "F.Cu") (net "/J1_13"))
 (segment (start 138.231 102.87) (end 138.236 102.865) (width 0.5) (layer "F.Cu") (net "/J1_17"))
 (segment (start 130.5 102.87) (end 138.231 102.87) (width 0.5) (layer "F.Cu") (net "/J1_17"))
 (segment (start 169.75 80.03) (end 161.121 80.03) (width 0.5) (layer "F.Cu") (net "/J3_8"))
 (segment (start 161.121 80.03) (end 161.096 80.005) (width 0.5) (layer "F.Cu") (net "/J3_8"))
 (segment (start 169.75 107.97) (end 161.121 107.97) (width 0.5) (layer "F.Cu") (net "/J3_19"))
 (segment (start 161.121 107.97) (end 161.096 107.945) (width 0.5) (layer "F.Cu") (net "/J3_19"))
 (segment (start 169.725 82.545) (end 169.75 82.57) (width 0.5) (layer "F.Cu") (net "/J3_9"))
 (segment (start 161.096 82.545) (end 169.725 82.545) (width 0.5) (layer "F.Cu") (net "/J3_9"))
 (segment (start 138.236 69.845) (end 130.505 69.845) (width 0.5) (layer "F.Cu") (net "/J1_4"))
 (segment (start 130.505 69.845) (end 130.5 69.85) (width 0.5) (layer "F.Cu") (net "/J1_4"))
 (segment (start 138.231 67.31) (end 138.236 67.305) (width 0.5) (layer "F.Cu") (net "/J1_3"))
 (segment (start 130.5 67.31) (end 138.231 67.31) (width 0.5) (layer "F.Cu") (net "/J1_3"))
 (segment (start 130.5 80.01) (end 138.231 80.01) (width 0.5) (layer "F.Cu") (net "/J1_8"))
 (segment (start 138.231 80.01) (end 138.236 80.005) (width 0.5) (layer "F.Cu") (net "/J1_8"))
 (segment (start 169.75 90.19) (end 161.121 90.19) (width 0.5) (layer "F.Cu") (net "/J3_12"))
 (segment (start 161.121 90.19) (end 161.096 90.165) (width 0.5) (layer "F.Cu") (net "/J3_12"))
 (segment (start 169.725 110.485) (end 169.75 110.51) (width 0.5) (layer "F.Cu") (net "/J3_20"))
 (segment (start 161.096 110.485) (end 169.725 110.485) (width 0.5) (layer "F.Cu") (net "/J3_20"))
 (segment (start 161.096 105.405) (end 169.725 105.405) (width 0.5) (layer "F.Cu") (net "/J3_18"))
 (segment (start 169.725 105.405) (end 169.75 105.43) (width 0.5) (layer "F.Cu") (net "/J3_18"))
 (segment (start 161.121 102.89) (end 161.096 102.865) (width 0.5) (layer "F.Cu") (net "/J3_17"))
 (segment (start 169.75 102.89) (end 161.121 102.89) (width 0.5) (layer "F.Cu") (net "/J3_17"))
 (segment (start 169.725 92.705) (end 169.75 92.73) (width 0.5) (layer "F.Cu") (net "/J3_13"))
 (segment (start 161.096 92.705) (end 169.725 92.705) (width 0.5) (layer "F.Cu") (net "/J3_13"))
 (segment (start 130.5 85.09) (end 138.231 85.09) (width 0.5) (layer "F.Cu") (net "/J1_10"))
 (segment (start 138.231 85.09) (end 138.236 85.085) (width 0.5) (layer "F.Cu") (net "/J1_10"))
 (segment (start 161.121 64.79) (end 161.096 64.765) (width 0.5) (layer "F.Cu") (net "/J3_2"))
 (segment (start 169.75 64.79) (end 161.121 64.79) (width 0.5) (layer "F.Cu") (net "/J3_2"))
 (segment (start 161.096 87.625) (end 169.725 87.625) (width 0.5) (layer "F.Cu") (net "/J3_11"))
 (segment (start 169.725 87.625) (end 169.75 87.65) (width 0.5) (layer "F.Cu") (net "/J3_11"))
 (segment (start 161.121 72.41) (end 161.096 72.385) (width 0.5) (layer "F.Cu") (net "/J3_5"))
 (segment (start 169.75 72.41) (end 161.121 72.41) (width 0.5) (layer "F.Cu") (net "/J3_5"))
 (segment (start 161.096 74.925) (end 169.725 74.925) (width 0.5) (layer "F.Cu") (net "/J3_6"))
 (segment (start 169.725 74.925) (end 169.75 74.95) (width 0.5) (layer "F.Cu") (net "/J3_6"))
 (segment (start 130.5 72.39) (end 138.231 72.39) (width 0.5) (layer "F.Cu") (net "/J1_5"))
 (segment (start 138.231 72.39) (end 138.236 72.385) (width 0.5) (layer "F.Cu") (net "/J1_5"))
 (segment (start 161.096 67.305) (end 169.725 67.305) (width 0.5) (layer "F.Cu") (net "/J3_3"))
 (segment (start 169.725 67.305) (end 169.75 67.33) (width 0.5) (layer "F.Cu") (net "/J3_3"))
 (segment (start 130.5 110.49) (end 138.231 110.49) (width 0.5) (layer "F.Cu") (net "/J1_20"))
 (segment (start 138.231 110.49) (end 138.236 110.485) (width 0.5) (layer "F.Cu") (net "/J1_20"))
 (segment (start 161.121 95.27) (end 161.096 95.245) (width 0.5) (layer "F.Cu") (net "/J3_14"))
 (segment (start 169.75 95.27) (end 161.121 95.27) (width 0.5) (layer "F.Cu") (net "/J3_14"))
 (segment (start 169.725 85.085) (end 169.75 85.11) (width 0.5) (layer "F.Cu") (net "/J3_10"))
 (segment (start 161.096 85.085) (end 169.725 85.085) (width 0.5) (layer "F.Cu") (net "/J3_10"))
 (segment (start 130.505 74.925) (end 130.5 74.93) (width 0.5) (layer "F.Cu") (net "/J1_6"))
 (segment (start 138.236 74.925) (end 130.505 74.925) (width 0.5) (layer "F.Cu") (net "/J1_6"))
 (segment (start 130.5 107.95) (end 138.231 107.95) (width 0.5) (layer "F.Cu") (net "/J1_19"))
 (segment (start 138.231 107.95) (end 138.236 107.945) (width 0.5) (layer "F.Cu") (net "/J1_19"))
 (segment (start 161.096 97.785) (end 169.725 97.785) (width 0.5) (layer "F.Cu") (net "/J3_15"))
 (segment (start 169.725 97.785) (end 169.75 97.81) (width 0.5) (layer "F.Cu") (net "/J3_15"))
 (segment (start 169.725 77.465) (end 169.75 77.49) (width 0.5) (layer "F.Cu") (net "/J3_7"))
 (segment (start 161.096 77.465) (end 169.725 77.465) (width 0.5) (layer "F.Cu") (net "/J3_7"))
 (segment (start 130.5 105.41) (end 138.231 105.41) (width 0.5) (layer "F.Cu") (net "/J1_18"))
 (segment (start 138.231 105.41) (end 138.236 105.405) (width 0.5) (layer "F.Cu") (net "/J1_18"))
 (segment (start 138.231 82.55) (end 138.236 82.545) (width 0.5) (layer "F.Cu") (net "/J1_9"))
 (segment (start 130.5 82.55) (end 138.231 82.55) (width 0.5) (layer "F.Cu") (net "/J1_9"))
 (segment (start 138.231 77.47) (end 138.236 77.465) (width 0.5) (layer "F.Cu") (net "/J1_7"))
 (segment (start 130.5 77.47) (end 138.231 77.47) (width 0.5) (layer "F.Cu") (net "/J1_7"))
 (segment (start 138.231 100.33) (end 138.236 100.325) (width 0.5) (layer "F.Cu") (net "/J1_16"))
 (segment (start 130.5 100.33) (end 138.231 100.33) (width 0.5) (layer "F.Cu") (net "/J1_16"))
 (segment (start 130.5 87.63) (end 138.231 87.63) (width 0.5) (layer "F.Cu") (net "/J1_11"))
 (segment (start 138.231 87.63) (end 138.236 87.625) (width 0.5) (layer "F.Cu") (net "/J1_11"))
 (segment (start 161.096 100.325) (end 169.725 100.325) (width 0.5) (layer "F.Cu") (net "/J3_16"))
 (segment (start 169.725 100.325) (end 169.75 100.35) (width 0.5) (layer "F.Cu") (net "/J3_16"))
 (segment (start 169.725 69.845) (end 169.75 69.87) (width 0.5) (layer "F.Cu") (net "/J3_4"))
 (segment (start 161.096 69.845) (end 169.725 69.845) (width 0.5) (layer "F.Cu") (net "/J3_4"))
 (segment (start 130.5 95.25) (end 138.231 95.25) (width 0.5) (layer "F.Cu") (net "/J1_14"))
 (segment (start 138.231 95.25) (end 138.236 95.245) (width 0.5) (layer "F.Cu") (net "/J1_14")))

